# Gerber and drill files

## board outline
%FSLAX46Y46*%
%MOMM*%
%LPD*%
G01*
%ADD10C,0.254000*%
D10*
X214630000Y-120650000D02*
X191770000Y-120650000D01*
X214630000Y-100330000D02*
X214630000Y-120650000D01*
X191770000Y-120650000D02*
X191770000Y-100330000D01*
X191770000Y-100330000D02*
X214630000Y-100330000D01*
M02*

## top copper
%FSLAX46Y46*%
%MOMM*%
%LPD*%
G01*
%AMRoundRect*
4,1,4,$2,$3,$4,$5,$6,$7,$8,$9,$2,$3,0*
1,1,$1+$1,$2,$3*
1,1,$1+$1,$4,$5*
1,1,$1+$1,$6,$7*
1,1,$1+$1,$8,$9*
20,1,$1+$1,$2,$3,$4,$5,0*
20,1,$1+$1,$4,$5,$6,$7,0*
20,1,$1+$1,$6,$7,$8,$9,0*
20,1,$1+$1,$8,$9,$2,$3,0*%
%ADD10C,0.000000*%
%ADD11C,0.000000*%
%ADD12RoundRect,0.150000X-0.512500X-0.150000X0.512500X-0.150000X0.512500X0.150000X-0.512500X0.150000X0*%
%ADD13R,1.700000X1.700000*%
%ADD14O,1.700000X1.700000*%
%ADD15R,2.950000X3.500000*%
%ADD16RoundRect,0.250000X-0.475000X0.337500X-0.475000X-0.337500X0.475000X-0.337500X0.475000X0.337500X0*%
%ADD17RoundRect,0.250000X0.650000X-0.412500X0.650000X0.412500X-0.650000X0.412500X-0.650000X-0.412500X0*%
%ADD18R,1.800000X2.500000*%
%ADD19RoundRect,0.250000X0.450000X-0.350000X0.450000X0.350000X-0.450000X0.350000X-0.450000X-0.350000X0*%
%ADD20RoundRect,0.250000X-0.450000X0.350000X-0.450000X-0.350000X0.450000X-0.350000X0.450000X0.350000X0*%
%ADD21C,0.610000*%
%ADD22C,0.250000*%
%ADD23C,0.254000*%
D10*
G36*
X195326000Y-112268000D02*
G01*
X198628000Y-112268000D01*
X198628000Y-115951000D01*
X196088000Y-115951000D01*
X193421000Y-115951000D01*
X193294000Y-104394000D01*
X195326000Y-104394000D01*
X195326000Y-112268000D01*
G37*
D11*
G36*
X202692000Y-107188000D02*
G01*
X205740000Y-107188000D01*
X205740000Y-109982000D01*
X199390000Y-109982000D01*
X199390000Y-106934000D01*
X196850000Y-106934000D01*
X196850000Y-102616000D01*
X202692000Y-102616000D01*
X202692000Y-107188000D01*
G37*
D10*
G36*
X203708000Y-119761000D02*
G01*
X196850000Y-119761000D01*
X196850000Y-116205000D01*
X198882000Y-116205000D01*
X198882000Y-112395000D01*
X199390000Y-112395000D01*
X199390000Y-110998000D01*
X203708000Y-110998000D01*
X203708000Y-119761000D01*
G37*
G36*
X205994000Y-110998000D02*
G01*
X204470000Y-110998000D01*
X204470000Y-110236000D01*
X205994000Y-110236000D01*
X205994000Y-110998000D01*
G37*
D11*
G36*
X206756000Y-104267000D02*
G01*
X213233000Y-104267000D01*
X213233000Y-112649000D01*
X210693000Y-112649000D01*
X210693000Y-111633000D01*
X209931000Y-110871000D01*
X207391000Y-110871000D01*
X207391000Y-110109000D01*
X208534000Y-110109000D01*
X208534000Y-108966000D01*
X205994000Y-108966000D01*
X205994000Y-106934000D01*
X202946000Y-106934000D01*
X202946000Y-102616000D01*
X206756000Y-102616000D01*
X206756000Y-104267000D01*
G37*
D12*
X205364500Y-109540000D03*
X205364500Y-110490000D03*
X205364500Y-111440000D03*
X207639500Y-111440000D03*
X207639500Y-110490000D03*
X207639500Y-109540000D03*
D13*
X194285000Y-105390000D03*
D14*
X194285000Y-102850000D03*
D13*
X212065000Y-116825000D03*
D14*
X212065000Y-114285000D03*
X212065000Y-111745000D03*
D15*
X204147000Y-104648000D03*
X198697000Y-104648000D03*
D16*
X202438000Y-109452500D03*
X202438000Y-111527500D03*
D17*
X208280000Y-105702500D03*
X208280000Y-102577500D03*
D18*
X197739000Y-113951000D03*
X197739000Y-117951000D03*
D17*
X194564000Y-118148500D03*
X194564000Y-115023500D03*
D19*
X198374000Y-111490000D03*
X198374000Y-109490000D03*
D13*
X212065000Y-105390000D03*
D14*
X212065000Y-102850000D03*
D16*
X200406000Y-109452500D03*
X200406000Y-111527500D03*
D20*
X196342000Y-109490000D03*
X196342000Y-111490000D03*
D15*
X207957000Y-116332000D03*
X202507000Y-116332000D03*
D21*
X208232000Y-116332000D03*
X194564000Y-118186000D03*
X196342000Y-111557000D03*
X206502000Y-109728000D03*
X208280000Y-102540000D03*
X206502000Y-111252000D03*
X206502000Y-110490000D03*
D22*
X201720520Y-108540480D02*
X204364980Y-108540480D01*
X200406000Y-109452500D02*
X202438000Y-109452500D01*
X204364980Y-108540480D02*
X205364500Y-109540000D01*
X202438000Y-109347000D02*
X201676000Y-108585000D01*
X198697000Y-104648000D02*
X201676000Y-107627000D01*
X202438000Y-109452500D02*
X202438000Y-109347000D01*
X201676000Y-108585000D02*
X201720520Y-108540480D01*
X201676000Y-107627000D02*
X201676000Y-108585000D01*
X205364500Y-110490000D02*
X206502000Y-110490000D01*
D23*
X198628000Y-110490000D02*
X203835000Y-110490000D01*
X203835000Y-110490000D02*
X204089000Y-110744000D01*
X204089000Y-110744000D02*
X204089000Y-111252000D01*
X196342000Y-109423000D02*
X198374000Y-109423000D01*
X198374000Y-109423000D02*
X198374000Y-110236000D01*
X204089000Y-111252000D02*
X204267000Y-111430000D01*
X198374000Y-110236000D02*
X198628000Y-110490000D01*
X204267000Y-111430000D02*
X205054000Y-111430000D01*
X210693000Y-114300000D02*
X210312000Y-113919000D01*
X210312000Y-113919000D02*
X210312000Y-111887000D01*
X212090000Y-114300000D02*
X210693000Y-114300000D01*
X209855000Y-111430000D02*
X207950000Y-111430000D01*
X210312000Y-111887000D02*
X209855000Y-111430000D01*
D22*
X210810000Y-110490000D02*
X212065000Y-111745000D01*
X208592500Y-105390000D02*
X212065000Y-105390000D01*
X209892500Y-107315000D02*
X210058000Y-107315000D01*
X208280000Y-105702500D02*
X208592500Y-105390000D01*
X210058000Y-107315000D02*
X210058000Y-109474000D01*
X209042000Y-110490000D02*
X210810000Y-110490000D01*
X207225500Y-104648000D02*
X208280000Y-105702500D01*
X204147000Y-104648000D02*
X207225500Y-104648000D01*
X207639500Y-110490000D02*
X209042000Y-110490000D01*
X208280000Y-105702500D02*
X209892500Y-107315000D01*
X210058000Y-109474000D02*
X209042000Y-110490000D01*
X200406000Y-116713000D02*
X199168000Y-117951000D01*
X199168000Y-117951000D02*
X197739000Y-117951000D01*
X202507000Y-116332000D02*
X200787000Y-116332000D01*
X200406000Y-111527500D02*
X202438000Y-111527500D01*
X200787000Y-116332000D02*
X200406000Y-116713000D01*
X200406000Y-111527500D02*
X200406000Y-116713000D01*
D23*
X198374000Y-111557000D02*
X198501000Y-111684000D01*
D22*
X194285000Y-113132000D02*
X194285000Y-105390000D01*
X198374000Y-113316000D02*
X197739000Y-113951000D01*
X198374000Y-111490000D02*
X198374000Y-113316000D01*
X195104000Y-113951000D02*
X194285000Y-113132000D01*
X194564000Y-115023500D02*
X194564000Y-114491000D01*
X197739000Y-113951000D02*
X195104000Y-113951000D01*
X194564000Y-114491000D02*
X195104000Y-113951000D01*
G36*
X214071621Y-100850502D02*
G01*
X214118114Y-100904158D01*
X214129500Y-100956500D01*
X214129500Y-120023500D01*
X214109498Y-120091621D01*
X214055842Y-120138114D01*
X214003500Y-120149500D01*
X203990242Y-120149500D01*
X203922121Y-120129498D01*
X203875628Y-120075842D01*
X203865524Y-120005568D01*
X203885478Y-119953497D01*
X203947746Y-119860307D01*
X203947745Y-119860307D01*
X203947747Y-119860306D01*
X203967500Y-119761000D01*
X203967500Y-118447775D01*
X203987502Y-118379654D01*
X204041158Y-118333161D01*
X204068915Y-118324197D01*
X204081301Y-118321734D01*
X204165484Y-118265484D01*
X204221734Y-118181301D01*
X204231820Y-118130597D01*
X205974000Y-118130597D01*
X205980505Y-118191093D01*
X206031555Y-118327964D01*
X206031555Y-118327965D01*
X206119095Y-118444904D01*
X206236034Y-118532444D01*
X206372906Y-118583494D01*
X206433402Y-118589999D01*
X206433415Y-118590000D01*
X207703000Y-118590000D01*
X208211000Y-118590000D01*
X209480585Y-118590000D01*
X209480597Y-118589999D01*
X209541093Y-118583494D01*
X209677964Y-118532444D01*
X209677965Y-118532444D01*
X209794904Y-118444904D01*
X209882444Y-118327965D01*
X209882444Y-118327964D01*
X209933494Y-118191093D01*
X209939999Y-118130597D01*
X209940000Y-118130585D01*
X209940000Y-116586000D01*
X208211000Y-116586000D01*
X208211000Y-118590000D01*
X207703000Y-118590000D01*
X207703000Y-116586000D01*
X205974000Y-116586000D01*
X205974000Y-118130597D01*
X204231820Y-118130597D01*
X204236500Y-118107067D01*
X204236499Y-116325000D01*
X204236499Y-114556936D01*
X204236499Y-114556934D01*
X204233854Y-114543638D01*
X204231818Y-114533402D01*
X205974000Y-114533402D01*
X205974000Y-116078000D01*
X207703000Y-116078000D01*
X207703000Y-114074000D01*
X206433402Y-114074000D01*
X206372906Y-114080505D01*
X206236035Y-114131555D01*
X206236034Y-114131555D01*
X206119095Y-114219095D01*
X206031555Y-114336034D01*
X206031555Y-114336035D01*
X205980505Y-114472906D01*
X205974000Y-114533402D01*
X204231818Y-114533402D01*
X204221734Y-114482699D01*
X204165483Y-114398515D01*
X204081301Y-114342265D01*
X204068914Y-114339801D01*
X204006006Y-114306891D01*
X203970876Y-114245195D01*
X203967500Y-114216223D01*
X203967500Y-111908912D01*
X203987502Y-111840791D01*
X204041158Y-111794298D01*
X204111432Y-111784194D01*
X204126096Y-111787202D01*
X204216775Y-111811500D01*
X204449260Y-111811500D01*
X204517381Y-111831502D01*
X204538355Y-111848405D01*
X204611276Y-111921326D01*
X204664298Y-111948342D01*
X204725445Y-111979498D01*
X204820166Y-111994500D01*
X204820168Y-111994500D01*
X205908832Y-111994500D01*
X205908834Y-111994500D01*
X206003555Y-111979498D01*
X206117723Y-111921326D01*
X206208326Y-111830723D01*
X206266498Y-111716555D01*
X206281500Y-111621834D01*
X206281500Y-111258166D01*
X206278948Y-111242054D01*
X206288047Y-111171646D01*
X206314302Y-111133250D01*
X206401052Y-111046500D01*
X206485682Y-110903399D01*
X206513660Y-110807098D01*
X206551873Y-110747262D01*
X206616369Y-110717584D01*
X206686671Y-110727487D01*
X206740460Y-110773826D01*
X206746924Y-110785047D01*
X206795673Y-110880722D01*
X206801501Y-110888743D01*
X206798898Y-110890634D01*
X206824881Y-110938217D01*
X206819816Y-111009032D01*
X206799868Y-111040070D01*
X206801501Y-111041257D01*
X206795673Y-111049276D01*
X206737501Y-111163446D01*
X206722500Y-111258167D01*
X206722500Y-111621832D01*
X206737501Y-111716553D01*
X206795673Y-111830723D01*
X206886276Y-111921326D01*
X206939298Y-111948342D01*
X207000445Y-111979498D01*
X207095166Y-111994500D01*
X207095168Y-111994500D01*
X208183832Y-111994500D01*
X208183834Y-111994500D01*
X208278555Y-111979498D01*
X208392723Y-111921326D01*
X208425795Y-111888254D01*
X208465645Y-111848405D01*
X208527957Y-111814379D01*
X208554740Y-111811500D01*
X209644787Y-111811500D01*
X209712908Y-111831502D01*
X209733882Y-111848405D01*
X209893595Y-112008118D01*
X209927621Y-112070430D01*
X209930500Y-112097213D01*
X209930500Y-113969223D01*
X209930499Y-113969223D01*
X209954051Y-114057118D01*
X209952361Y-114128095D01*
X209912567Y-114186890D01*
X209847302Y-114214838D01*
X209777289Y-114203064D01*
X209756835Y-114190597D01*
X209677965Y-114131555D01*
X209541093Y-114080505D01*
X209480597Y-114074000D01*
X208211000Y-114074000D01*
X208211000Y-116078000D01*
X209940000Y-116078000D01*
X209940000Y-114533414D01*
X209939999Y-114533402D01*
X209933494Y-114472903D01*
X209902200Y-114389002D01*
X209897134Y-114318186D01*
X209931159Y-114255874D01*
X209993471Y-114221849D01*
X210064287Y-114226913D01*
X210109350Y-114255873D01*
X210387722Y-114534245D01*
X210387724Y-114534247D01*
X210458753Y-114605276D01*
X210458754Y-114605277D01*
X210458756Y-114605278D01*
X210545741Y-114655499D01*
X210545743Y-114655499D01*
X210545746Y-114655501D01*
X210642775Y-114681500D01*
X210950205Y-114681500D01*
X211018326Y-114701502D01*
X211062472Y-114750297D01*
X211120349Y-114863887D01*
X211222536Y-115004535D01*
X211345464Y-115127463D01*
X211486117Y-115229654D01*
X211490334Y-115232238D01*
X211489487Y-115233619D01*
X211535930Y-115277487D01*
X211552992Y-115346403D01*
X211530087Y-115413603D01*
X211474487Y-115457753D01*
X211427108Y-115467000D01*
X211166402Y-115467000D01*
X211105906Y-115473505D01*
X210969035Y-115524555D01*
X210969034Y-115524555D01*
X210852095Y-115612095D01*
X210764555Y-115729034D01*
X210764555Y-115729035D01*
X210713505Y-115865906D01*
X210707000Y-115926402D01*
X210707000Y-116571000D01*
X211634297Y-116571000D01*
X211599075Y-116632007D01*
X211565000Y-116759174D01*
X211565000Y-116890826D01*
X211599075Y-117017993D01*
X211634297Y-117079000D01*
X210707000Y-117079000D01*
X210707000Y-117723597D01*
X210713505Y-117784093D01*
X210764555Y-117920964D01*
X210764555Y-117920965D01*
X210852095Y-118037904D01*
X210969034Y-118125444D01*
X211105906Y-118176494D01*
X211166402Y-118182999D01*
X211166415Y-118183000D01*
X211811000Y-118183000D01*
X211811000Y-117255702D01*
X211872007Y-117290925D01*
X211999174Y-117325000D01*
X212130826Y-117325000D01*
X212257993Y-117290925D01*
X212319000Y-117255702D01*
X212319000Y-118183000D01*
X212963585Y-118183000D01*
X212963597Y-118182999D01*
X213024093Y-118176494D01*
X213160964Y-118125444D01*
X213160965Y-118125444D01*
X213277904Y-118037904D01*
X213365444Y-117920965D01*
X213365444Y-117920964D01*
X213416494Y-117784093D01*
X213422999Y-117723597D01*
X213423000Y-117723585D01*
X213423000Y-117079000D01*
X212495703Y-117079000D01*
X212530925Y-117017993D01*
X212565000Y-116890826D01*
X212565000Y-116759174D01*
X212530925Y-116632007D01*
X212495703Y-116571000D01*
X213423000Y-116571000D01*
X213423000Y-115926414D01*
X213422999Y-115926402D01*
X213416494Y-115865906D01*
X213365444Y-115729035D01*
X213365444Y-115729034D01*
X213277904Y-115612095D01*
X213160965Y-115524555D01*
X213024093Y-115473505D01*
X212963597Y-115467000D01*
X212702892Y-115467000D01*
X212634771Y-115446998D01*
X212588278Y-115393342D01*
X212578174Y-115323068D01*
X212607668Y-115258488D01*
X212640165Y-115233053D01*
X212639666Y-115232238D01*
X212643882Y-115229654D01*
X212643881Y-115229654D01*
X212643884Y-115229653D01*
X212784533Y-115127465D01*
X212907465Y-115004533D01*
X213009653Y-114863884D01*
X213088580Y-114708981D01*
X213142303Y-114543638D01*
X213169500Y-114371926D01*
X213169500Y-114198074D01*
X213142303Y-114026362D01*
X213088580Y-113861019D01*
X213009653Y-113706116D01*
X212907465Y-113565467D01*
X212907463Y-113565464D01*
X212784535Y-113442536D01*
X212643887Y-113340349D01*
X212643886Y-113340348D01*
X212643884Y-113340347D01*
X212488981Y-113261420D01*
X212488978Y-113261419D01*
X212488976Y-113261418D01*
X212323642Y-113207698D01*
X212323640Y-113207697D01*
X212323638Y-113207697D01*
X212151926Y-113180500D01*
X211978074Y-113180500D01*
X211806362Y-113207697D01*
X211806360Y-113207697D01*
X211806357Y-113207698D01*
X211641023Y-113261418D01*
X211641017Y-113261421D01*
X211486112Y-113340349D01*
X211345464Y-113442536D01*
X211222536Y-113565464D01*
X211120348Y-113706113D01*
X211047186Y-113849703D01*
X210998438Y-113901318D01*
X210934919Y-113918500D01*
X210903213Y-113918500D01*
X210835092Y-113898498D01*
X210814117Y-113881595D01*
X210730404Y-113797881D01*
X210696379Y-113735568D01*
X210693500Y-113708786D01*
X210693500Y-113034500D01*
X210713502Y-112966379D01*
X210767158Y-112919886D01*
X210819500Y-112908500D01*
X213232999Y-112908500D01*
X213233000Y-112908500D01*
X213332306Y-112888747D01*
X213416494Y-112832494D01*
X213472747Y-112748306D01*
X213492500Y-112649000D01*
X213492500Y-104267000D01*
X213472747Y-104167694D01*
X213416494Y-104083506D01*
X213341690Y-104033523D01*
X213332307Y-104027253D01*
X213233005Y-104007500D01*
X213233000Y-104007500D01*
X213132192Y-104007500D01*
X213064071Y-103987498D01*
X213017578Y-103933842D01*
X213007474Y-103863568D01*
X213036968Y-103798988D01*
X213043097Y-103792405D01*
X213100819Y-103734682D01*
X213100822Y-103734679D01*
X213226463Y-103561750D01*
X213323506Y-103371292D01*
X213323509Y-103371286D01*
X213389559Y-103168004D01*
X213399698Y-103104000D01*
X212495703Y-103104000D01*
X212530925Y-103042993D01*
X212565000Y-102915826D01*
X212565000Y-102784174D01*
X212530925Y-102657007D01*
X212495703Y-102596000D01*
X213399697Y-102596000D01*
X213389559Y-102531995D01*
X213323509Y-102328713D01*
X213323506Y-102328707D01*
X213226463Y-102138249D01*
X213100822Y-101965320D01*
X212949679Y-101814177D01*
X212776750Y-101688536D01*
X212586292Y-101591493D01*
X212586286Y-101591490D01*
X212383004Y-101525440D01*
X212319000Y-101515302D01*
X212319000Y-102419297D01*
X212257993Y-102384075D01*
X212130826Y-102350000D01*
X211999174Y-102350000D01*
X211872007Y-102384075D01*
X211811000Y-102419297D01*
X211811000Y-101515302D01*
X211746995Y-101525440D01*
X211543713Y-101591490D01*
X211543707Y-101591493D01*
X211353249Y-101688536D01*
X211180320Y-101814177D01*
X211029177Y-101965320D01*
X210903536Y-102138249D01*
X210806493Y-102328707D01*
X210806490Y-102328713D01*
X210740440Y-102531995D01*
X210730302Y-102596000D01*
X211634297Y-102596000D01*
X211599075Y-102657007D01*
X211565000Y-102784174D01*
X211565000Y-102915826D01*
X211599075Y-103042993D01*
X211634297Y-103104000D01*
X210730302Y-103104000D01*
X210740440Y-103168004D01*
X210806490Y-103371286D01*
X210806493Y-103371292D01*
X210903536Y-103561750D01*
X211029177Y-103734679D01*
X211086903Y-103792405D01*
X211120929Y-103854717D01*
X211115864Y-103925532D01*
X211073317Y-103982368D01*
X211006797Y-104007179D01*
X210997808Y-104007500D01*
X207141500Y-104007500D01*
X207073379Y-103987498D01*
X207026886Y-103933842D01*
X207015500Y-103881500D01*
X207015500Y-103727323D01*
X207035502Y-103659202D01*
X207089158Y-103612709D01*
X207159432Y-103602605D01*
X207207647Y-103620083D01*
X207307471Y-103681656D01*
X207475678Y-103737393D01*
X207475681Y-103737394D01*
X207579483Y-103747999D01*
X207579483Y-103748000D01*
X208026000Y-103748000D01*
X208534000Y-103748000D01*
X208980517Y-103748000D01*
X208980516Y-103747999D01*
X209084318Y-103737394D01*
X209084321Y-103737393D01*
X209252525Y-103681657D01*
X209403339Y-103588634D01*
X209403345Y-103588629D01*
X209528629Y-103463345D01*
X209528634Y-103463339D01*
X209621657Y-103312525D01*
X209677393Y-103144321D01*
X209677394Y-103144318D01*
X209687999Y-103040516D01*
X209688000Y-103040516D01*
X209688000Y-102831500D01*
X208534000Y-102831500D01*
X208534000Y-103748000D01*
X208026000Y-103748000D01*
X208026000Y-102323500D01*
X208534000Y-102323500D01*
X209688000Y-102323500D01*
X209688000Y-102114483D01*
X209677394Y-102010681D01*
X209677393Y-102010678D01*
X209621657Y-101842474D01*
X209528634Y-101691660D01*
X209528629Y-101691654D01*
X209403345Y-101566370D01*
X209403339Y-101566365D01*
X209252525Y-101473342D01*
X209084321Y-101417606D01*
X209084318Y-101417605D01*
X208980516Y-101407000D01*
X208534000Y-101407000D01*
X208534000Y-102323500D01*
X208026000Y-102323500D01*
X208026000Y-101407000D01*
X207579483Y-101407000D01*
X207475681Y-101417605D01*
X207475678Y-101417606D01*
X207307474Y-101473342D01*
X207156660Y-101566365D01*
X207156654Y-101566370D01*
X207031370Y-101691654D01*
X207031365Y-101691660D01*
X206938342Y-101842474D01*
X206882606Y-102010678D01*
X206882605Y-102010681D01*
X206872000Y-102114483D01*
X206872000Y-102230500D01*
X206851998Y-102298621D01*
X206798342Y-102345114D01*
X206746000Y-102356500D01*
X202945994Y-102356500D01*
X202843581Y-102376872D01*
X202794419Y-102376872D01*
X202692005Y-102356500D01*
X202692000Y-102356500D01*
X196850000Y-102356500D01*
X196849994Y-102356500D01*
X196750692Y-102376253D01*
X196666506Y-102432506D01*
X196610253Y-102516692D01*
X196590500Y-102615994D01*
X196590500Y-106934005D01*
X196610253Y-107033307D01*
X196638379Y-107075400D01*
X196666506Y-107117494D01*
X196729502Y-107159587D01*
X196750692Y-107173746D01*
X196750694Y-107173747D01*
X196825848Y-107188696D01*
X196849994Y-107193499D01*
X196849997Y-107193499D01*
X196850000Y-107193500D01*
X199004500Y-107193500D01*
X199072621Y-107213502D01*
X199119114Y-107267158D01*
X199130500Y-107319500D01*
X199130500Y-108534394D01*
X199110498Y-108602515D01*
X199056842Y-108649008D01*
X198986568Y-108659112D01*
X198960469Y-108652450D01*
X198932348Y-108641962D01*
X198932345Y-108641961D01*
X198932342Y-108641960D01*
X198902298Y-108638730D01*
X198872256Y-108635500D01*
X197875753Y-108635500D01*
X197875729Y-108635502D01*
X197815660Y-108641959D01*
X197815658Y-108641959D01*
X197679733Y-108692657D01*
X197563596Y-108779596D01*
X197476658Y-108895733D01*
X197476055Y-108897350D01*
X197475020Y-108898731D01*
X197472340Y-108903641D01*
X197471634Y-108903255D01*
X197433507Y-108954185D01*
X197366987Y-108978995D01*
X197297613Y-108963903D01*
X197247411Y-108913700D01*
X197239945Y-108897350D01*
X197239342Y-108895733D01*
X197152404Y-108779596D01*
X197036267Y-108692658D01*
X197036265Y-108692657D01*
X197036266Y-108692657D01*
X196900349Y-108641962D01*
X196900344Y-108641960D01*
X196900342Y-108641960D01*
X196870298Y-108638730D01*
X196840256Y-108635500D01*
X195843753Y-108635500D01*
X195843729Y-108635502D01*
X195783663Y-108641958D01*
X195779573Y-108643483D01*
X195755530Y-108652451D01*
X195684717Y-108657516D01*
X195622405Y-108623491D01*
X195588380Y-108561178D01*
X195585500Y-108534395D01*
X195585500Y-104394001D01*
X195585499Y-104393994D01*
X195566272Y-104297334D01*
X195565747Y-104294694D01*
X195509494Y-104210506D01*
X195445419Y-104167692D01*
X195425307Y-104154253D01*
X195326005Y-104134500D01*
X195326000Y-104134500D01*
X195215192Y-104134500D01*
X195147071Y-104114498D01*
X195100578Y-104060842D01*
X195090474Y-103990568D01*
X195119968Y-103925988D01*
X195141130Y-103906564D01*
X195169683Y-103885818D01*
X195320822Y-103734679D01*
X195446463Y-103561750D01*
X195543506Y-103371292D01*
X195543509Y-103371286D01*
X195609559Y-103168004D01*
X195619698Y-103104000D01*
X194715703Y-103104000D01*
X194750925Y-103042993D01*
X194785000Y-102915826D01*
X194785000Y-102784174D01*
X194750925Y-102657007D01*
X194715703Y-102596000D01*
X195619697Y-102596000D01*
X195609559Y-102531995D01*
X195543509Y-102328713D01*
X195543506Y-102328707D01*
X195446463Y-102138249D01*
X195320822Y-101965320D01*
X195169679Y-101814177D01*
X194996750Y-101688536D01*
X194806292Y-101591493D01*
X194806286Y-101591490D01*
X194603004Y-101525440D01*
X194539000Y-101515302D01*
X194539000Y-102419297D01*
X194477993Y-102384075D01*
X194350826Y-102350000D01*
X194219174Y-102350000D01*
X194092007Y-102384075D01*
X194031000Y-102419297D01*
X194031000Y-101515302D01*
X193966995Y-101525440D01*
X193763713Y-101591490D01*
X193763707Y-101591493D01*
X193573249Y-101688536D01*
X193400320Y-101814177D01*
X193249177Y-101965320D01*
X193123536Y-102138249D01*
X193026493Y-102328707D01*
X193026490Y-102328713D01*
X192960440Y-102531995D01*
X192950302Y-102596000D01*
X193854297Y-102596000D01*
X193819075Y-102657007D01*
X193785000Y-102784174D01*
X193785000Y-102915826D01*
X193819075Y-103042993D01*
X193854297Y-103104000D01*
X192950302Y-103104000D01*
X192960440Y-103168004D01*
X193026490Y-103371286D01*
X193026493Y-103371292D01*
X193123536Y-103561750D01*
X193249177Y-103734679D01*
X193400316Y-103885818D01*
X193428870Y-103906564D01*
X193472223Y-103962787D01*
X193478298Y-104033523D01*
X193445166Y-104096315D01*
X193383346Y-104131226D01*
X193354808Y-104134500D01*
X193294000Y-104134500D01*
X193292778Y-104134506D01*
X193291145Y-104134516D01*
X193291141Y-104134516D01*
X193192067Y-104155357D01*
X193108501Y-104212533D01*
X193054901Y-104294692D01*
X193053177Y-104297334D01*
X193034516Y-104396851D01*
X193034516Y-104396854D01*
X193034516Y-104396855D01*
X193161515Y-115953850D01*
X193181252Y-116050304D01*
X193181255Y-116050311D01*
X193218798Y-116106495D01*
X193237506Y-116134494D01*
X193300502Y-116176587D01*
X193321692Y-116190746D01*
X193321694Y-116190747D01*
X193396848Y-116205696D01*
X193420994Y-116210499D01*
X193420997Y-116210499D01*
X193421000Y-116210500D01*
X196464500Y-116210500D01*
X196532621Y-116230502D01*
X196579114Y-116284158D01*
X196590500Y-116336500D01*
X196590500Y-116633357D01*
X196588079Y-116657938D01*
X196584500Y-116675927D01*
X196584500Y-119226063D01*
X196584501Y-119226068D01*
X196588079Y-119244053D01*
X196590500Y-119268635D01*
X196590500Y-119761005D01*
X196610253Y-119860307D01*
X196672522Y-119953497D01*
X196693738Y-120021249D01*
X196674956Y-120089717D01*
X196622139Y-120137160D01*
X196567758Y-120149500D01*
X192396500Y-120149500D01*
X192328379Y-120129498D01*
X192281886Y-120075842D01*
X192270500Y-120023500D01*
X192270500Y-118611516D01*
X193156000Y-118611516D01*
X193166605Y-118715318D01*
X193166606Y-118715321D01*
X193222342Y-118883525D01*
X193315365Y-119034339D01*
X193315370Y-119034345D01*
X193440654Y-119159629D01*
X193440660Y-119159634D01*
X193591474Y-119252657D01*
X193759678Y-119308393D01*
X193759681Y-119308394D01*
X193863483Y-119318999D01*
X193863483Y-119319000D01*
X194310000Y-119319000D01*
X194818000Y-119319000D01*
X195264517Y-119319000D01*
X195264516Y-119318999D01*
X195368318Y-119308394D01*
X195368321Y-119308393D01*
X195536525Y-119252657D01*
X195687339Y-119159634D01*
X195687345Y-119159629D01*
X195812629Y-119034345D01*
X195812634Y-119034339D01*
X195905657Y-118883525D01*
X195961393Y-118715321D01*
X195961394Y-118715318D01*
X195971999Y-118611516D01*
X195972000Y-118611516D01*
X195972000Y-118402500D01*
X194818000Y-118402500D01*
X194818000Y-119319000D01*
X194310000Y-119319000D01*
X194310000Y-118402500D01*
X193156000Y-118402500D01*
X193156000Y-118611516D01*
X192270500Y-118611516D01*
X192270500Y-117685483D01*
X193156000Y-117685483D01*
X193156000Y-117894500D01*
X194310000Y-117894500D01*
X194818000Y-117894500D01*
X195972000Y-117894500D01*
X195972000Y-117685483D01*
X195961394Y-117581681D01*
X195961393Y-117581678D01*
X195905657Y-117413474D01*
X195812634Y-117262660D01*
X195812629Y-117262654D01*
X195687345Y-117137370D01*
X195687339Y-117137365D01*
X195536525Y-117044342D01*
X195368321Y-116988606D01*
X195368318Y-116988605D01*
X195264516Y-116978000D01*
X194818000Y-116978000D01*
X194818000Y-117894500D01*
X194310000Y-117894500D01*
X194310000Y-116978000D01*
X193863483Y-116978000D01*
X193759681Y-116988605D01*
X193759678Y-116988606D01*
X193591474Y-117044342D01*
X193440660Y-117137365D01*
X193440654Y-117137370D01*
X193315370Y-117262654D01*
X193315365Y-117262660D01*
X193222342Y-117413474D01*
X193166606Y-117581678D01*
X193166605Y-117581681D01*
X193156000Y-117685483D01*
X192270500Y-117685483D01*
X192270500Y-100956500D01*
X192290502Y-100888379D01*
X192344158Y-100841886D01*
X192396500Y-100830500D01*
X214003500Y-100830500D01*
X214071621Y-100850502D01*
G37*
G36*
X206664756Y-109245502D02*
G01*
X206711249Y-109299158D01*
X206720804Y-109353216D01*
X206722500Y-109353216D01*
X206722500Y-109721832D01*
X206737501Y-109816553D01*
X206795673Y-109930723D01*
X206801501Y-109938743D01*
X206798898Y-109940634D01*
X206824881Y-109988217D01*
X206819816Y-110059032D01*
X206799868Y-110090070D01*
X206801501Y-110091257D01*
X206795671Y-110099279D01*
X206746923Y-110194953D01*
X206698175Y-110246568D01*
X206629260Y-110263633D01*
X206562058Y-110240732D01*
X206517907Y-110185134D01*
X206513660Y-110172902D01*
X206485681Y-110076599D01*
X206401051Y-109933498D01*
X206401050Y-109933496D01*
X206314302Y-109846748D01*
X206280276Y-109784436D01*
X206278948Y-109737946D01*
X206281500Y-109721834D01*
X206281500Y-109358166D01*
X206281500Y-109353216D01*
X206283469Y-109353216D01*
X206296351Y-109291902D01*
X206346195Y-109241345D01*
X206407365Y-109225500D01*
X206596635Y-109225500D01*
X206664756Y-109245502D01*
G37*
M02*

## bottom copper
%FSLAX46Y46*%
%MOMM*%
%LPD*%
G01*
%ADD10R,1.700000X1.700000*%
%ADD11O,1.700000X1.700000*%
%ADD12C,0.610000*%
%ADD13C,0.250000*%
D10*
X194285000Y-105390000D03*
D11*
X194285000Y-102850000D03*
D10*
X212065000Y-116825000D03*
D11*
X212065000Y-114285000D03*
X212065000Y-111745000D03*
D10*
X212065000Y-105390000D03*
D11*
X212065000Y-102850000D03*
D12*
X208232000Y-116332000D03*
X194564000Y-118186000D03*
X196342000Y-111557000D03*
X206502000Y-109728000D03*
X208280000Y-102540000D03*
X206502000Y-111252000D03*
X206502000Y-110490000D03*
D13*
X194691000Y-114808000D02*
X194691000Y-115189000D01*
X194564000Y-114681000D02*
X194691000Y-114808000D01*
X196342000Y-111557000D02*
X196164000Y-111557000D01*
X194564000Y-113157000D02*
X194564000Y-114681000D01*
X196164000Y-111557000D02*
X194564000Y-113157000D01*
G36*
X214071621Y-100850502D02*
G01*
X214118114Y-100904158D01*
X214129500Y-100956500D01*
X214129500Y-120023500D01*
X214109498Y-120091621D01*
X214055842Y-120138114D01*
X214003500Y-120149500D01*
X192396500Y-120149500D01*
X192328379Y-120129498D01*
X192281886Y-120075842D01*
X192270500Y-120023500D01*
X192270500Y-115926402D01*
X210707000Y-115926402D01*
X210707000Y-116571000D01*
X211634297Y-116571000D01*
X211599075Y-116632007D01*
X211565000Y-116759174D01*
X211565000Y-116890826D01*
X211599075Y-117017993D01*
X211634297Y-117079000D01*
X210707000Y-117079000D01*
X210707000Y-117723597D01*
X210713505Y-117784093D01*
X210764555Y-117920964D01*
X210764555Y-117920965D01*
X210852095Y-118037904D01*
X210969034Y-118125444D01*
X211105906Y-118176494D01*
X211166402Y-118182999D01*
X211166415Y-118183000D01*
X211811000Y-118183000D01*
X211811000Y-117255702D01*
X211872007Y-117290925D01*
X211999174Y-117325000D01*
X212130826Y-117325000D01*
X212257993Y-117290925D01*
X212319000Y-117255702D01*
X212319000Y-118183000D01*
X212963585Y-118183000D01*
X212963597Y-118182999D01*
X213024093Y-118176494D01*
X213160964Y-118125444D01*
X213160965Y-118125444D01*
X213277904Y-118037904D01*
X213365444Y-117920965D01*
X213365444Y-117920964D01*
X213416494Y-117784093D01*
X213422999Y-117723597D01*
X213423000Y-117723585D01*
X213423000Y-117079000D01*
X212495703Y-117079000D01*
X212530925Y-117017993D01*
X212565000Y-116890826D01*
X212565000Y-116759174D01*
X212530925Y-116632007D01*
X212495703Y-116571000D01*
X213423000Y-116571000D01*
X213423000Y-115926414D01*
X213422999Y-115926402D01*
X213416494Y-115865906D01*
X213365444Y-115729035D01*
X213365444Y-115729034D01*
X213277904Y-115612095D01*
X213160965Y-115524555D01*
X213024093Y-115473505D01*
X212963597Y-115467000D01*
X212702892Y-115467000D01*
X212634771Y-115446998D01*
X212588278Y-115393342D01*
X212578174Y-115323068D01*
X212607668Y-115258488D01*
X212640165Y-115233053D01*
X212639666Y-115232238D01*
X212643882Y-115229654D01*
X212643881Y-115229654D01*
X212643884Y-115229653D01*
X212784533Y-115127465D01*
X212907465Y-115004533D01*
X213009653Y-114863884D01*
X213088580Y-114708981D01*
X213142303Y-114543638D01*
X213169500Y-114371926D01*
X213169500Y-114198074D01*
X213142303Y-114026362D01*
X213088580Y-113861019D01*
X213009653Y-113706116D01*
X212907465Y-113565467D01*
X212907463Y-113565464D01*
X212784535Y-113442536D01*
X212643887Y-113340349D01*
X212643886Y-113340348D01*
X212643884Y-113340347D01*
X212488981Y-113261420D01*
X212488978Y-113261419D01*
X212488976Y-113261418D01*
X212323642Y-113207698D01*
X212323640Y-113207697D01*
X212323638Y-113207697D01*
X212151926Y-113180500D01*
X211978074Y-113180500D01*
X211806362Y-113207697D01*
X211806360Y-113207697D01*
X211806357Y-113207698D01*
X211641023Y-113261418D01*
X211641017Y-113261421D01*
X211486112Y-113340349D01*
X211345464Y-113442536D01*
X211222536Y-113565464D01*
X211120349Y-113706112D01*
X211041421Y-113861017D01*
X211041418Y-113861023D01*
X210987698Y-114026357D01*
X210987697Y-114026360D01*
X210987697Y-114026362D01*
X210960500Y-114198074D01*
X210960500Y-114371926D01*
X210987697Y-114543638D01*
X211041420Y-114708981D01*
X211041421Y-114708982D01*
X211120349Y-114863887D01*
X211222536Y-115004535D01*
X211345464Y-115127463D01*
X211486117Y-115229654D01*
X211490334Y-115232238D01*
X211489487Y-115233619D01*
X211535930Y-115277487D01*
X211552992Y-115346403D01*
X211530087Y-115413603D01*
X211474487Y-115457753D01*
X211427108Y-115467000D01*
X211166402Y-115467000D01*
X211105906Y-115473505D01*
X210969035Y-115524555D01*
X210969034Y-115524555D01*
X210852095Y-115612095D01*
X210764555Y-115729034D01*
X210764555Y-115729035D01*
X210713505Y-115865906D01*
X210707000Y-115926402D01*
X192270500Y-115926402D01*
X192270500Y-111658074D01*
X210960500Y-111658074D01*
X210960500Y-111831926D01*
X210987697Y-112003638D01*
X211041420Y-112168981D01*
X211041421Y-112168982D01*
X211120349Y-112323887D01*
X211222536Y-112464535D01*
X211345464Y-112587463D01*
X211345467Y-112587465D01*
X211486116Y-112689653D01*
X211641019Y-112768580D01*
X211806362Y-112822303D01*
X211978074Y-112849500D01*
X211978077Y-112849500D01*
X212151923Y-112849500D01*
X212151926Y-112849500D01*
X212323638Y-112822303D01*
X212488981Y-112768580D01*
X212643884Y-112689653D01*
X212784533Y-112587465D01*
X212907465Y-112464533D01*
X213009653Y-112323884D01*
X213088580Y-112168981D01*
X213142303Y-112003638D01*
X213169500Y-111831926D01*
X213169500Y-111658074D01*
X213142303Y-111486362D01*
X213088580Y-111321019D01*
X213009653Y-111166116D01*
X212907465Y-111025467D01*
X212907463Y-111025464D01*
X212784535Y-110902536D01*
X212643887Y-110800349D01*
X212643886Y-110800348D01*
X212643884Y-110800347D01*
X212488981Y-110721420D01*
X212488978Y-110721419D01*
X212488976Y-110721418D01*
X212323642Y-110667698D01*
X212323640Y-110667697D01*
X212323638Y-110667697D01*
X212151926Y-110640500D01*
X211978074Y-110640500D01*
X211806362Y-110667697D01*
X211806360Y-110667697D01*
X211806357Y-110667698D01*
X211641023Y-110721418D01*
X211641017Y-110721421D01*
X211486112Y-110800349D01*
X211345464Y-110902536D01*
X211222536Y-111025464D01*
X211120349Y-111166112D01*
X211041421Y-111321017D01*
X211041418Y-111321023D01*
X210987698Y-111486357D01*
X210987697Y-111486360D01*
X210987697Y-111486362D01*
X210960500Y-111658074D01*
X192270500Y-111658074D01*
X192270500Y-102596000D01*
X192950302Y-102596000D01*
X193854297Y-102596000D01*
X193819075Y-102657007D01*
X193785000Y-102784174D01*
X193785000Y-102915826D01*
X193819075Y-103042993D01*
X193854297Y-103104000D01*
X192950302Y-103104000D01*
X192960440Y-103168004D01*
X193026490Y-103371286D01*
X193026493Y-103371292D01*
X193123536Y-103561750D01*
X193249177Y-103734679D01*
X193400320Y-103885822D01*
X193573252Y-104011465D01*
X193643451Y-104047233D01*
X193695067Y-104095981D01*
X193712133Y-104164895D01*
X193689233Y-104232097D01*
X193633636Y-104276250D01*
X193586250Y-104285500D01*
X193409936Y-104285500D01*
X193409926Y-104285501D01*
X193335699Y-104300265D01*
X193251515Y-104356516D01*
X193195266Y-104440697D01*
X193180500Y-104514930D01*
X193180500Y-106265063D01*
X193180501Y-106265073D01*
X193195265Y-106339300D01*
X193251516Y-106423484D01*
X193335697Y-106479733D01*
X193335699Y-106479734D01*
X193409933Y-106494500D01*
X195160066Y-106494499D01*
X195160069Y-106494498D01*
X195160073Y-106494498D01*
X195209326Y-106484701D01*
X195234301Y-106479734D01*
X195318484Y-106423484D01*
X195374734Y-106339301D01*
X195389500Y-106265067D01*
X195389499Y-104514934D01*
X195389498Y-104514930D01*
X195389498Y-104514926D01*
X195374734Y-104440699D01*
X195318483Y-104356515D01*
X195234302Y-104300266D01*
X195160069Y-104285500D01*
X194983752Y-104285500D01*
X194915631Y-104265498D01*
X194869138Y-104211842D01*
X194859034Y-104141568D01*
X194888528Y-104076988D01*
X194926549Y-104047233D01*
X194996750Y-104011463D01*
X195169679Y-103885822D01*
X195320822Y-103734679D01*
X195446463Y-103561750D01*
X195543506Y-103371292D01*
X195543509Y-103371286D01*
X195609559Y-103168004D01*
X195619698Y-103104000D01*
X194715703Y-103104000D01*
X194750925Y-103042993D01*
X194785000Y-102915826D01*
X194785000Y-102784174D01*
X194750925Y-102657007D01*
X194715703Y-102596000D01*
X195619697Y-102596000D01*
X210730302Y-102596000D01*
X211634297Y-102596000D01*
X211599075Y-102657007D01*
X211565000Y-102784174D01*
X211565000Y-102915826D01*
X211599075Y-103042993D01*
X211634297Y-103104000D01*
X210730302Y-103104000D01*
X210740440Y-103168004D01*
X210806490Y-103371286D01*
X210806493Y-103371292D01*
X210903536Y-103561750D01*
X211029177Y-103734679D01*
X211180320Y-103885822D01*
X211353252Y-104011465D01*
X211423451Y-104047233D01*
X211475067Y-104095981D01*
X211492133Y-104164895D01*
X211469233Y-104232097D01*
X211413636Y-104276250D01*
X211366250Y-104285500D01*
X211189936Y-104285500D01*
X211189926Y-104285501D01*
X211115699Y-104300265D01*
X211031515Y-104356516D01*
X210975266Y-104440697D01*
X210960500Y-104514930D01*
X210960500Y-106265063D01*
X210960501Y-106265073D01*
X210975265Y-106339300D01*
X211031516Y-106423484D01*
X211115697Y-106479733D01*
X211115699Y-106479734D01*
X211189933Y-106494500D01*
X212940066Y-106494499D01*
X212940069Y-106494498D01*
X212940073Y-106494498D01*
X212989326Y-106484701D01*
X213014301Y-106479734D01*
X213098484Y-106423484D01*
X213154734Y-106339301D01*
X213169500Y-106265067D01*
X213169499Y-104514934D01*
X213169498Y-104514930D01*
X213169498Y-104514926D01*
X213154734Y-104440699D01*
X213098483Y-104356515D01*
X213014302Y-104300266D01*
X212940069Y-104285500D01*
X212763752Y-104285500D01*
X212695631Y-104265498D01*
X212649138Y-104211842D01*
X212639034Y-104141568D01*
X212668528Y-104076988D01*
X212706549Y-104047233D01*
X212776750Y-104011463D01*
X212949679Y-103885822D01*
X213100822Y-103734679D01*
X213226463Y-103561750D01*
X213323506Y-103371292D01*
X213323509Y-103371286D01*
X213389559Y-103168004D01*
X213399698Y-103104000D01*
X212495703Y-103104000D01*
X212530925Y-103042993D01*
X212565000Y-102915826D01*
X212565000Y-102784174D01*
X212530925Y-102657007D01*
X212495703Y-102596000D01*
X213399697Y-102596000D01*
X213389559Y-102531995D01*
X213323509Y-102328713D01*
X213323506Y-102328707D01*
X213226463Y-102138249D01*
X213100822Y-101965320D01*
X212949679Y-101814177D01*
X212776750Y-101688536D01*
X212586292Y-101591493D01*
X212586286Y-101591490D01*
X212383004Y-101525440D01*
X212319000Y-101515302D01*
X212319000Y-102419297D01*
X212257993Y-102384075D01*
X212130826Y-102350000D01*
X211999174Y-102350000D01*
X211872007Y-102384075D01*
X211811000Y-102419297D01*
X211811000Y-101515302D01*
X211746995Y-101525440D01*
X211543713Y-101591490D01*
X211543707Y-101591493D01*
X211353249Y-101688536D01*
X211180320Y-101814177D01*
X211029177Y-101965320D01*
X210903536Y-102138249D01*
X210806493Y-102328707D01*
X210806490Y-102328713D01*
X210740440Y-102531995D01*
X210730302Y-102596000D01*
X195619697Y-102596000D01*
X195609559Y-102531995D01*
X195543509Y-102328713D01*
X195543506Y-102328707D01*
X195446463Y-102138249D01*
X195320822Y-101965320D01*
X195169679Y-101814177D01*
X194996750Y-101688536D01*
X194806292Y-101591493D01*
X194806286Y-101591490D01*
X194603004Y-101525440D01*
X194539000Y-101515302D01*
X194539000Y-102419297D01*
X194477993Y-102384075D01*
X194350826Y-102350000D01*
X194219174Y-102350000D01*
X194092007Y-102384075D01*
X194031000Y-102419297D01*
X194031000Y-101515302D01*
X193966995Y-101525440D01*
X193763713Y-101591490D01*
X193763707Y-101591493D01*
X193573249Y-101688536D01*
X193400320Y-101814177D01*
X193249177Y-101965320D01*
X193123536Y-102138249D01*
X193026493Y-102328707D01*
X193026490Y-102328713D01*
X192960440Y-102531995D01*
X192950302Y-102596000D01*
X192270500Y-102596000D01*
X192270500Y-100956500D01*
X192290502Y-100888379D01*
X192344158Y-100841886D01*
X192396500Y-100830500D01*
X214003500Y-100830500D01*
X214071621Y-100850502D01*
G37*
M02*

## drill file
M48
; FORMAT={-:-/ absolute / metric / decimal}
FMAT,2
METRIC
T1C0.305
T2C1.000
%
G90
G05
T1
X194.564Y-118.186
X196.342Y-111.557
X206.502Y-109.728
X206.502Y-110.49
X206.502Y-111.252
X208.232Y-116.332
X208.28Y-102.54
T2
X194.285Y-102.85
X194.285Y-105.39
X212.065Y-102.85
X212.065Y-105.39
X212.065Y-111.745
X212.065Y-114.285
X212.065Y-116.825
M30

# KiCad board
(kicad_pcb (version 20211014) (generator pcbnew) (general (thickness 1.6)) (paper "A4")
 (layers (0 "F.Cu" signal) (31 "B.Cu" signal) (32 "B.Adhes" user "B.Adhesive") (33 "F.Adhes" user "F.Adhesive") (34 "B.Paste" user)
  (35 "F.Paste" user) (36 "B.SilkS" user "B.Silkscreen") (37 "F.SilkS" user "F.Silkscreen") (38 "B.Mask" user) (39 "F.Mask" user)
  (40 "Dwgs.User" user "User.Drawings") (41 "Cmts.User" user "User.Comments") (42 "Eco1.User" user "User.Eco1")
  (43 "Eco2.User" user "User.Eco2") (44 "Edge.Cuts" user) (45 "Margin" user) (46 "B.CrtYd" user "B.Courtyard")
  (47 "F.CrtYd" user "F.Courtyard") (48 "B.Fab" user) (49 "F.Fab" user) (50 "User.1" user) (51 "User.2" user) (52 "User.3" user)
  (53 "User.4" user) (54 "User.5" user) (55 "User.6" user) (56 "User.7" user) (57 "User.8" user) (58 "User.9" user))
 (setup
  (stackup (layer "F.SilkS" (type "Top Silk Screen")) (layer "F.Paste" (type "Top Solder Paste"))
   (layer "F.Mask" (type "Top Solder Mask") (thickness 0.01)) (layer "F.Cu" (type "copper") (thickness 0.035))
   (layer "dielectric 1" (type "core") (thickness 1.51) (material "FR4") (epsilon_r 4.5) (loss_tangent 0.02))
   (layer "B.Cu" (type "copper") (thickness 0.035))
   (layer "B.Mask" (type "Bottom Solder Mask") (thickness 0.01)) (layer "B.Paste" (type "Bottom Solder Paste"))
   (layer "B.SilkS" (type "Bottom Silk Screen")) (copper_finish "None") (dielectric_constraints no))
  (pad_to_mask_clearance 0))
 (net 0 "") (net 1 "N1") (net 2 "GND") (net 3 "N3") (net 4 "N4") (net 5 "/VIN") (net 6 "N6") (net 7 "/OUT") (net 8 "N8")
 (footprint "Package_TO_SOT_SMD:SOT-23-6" (layer "F.Cu") (at 206.502 110.49)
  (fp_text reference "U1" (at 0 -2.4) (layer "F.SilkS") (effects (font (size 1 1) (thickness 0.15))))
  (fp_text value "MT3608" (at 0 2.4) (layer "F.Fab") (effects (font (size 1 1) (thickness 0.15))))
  (pad "1" smd roundrect locked (at -1.1375 -0.95) (size 1.325 0.6) (layers "F.Cu" "F.Paste" "F.Mask") (roundrect_rratio 0.25) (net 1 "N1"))
  (pad "2" smd roundrect locked (at -1.1375 0) (size 1.325 0.6) (layers "F.Cu" "F.Paste" "F.Mask") (roundrect_rratio 0.25) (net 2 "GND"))
  (pad "3" smd roundrect locked (at -1.1375 0.95) (size 1.325 0.6) (layers "F.Cu" "F.Paste" "F.Mask") (roundrect_rratio 0.25) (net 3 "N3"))
  (pad "4" smd roundrect locked (at 1.1375 0.95) (size 1.325 0.6) (layers "F.Cu" "F.Paste" "F.Mask") (roundrect_rratio 0.25) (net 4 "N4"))
  (pad "5" smd roundrect locked (at 1.1375 0) (size 1.325 0.6) (layers "F.Cu" "F.Paste" "F.Mask") (roundrect_rratio 0.25) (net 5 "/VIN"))
  (pad "6" smd roundrect locked (at 1.1375 -0.95) (size 1.325 0.6) (layers "F.Cu" "F.Paste" "F.Mask") (roundrect_rratio 0.25) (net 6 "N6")))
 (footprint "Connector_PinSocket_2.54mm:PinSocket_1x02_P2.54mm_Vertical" (layer "F.Cu") (at 194.285 105.39 180)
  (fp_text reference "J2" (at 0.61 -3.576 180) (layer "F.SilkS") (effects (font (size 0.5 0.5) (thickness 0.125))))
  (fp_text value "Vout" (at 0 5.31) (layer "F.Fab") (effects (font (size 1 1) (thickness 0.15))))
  (pad "1" thru_hole rect locked (at 0 0 180) (size 1.7 1.7) (drill 1) (layers *.Cu *.Mask) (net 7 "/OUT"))
  (pad "2" thru_hole oval locked (at 0 2.54 180) (size 1.7 1.7) (drill 1) (layers *.Cu *.Mask) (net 2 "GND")))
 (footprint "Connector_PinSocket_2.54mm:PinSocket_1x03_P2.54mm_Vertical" (layer "F.Cu") (at 212.065 116.825 180)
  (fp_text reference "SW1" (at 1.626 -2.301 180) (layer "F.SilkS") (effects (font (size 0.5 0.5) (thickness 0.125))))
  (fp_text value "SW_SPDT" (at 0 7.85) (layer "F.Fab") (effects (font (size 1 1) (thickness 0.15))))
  (pad "1" thru_hole rect locked (at 0 0 180) (size 1.7 1.7) (drill 1) (layers *.Cu *.Mask) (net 2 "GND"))
  (pad "2" thru_hole oval locked (at 0 2.54 180) (size 1.7 1.7) (drill 1) (layers *.Cu *.Mask) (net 4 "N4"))
  (pad "3" thru_hole oval locked (at 0 5.08 180) (size 1.7 1.7) (drill 1) (layers *.Cu *.Mask) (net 5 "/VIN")))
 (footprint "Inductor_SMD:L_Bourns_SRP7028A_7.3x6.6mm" (layer "F.Cu") (at 201.422 104.648 180)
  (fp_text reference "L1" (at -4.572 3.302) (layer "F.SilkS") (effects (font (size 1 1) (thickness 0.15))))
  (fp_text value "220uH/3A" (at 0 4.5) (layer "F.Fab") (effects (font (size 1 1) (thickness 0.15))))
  (pad "1" smd rect locked (at -2.725 0 180) (size 2.95 3.5) (layers "F.Cu" "F.Paste" "F.Mask") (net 5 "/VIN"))
  (pad "2" smd rect locked (at 2.725 0 180) (size 2.95 3.5) (layers "F.Cu" "F.Paste" "F.Mask") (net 1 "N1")))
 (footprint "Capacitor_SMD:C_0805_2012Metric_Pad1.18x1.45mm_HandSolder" (layer "F.Cu") (at 202.438 110.49 -90)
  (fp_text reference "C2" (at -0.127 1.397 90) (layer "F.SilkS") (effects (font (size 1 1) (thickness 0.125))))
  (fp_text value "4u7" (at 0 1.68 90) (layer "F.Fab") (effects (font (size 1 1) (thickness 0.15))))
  (pad "1" smd roundrect locked (at -1.0375 0 270) (size 1.175 1.45) (layers "F.Cu" "F.Paste" "F.Mask") (roundrect_rratio 0.212766)
   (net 1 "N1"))
  (pad "2" smd roundrect locked (at 1.0375 0 270) (size 1.175 1.45) (layers "F.Cu" "F.Paste" "F.Mask") (roundrect_rratio 0.212766)
   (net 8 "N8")))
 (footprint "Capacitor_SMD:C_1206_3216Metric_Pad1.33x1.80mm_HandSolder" (layer "F.Cu") (at 208.28 104.14 90)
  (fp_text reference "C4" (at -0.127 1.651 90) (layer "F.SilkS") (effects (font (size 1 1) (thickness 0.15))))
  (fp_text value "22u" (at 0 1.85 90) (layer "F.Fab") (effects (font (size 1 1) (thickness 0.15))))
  (pad "1" smd roundrect locked (at -1.5625 0 90) (size 1.325 1.8) (layers "F.Cu" "F.Paste" "F.Mask") (roundrect_rratio 0.188679)
   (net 5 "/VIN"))
  (pad "2" smd roundrect locked (at 1.5625 0 90) (size 1.325 1.8) (layers "F.Cu" "F.Paste" "F.Mask") (roundrect_rratio 0.188679)
   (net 2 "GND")))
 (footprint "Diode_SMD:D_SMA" (layer "F.Cu") (at 197.739 115.951 -90)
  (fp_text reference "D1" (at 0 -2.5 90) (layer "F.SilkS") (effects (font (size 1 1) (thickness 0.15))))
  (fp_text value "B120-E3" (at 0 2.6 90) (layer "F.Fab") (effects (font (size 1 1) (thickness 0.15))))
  (pad "1" smd rect locked (at -2 0 270) (size 2.5 1.8) (layers "F.Cu" "F.Paste" "F.Mask") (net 7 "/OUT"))
  (pad "2" smd rect locked (at 2 0 270) (size 2.5 1.8) (layers "F.Cu" "F.Paste" "F.Mask") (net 8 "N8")))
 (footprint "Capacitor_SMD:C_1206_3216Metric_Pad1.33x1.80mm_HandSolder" (layer "F.Cu") (at 194.564 116.586 90)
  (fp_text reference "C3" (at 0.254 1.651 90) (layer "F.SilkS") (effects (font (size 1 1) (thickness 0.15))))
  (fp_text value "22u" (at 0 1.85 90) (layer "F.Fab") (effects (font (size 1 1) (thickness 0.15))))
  (pad "1" smd roundrect locked (at -1.5625 0 90) (size 1.325 1.8) (layers "F.Cu" "F.Paste" "F.Mask") (roundrect_rratio 0.188679)
   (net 2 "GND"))
  (pad "2" smd roundrect locked (at 1.5625 0 90) (size 1.325 1.8) (layers "F.Cu" "F.Paste" "F.Mask") (roundrect_rratio 0.188679)
   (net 7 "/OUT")))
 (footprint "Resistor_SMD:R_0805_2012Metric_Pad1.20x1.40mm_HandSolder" (layer "F.Cu") (at 198.374 110.49 90)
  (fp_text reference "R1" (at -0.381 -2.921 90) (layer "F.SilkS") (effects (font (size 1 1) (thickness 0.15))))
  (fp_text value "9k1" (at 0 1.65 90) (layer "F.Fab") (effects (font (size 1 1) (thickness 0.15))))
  (pad "1" smd roundrect locked (at -1 0 90) (size 1.2 1.4) (layers "F.Cu" "F.Paste" "F.Mask") (roundrect_rratio 0.208333) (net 7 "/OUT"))
  (pad "2" smd roundrect locked (at 1 0 90) (size 1.2 1.4) (layers "F.Cu" "F.Paste" "F.Mask") (roundrect_rratio 0.208333) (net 3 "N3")))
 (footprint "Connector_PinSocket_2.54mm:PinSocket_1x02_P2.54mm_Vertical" (layer "F.Cu") (at 212.065 105.39 180)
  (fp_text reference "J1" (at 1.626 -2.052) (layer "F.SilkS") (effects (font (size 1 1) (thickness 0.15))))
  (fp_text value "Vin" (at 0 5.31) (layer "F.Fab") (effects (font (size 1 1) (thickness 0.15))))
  (pad "1" thru_hole rect locked (at 0 0 180) (size 1.7 1.7) (drill 1) (layers *.Cu *.Mask) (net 5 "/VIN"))
  (pad "2" thru_hole oval locked (at 0 2.54 180) (size 1.7 1.7) (drill 1) (layers *.Cu *.Mask) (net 2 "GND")))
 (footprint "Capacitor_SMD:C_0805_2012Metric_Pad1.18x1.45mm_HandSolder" (layer "F.Cu") (at 200.406 110.49 -90)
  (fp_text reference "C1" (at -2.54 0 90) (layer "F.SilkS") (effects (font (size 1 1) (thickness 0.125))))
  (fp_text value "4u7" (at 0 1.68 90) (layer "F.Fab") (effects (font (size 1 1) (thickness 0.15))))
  (pad "1" smd roundrect locked (at -1.0375 0 270) (size 1.175 1.45) (layers "F.Cu" "F.Paste" "F.Mask") (roundrect_rratio 0.212766)
   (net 1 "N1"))
  (pad "2" smd roundrect locked (at 1.0375 0 270) (size 1.175 1.45) (layers "F.Cu" "F.Paste" "F.Mask") (roundrect_rratio 0.212766)
   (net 8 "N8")))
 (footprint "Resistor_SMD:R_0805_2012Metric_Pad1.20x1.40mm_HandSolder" (layer "F.Cu") (at 196.342 110.49 -90)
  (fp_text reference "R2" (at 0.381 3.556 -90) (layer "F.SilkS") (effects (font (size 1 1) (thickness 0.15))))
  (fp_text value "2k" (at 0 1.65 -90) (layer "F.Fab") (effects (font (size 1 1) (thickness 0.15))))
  (pad "1" smd roundrect locked (at -1 0 270) (size 1.2 1.4) (layers "F.Cu" "F.Paste" "F.Mask") (roundrect_rratio 0.208333) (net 3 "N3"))
  (pad "2" smd roundrect locked (at 1 0 270) (size 1.2 1.4) (layers "F.Cu" "F.Paste" "F.Mask") (roundrect_rratio 0.208333) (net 2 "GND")))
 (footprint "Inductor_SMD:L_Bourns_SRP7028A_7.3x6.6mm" (layer "F.Cu") (at 205.232 116.332 180)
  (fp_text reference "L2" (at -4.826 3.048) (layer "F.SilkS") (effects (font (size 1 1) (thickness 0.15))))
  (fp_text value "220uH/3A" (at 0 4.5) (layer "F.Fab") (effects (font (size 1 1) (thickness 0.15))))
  (pad "1" smd rect locked (at -2.725 0 180) (size 2.95 3.5) (layers "F.Cu" "F.Paste" "F.Mask") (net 2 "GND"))
  (pad "2" smd rect locked (at 2.725 0 180) (size 2.95 3.5) (layers "F.Cu" "F.Paste" "F.Mask") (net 8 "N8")))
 (gr_poly
  (pts (xy 198.628 115.951) (xy 198.628 112.268) (xy 195.326 112.268) (xy 195.326 104.394) (xy 193.294 104.394) (xy 193.421 115.951)
   (xy 196.088 115.951))
  (layer "F.Cu") (width 0) (fill solid))
 (gr_poly
  (pts (xy 196.85 102.616) (xy 196.85 106.934) (xy 199.39 106.934) (xy 199.39 109.982) (xy 205.74 109.982) (xy 205.74 107.188)
   (xy 202.692 107.188) (xy 202.692 102.616))
  (layer "F.Cu") (width 0) (fill solid))
 (gr_poly
  (pts (xy 199.39 110.998) (xy 199.39 112.395) (xy 198.882 112.395) (xy 198.882 116.205) (xy 196.85 116.205) (xy 196.85 119.761)
   (xy 203.708 119.761) (xy 203.708 110.998))
  (layer "F.Cu") (width 0) (fill solid))
 (gr_poly (pts (xy 204.47 110.236) (xy 205.994 110.236) (xy 205.994 110.998) (xy 204.47 110.998)) (layer "F.Cu") (width 0) (fill solid))
 (gr_poly
  (pts (xy 213.233 104.267) (xy 206.756 104.267) (xy 206.756 102.616) (xy 202.946 102.616) (xy 202.946 106.934) (xy 205.994 106.934)
   (xy 205.994 108.966) (xy 208.534 108.966) (xy 208.534 110.109) (xy 207.391 110.109) (xy 207.391 110.871) (xy 209.931 110.871)
   (xy 210.693 111.633) (xy 210.693 112.649) (xy 213.233 112.649))
  (layer "F.Cu") (width 0) (fill solid))
 (gr_line (start 214.63 120.65) (end 191.77 120.65) (layer "Edge.Cuts") (width 0.254))
 (gr_line (start 214.63 100.33) (end 214.63 120.65) (layer "Edge.Cuts") (width 0.254))
 (gr_line (start 191.77 120.65) (end 191.77 100.33) (layer "Edge.Cuts") (width 0.254))
 (gr_line (start 191.77 100.33) (end 214.63 100.33) (layer "Edge.Cuts") (width 0.254))
 (segment (start 201.72052 108.54048) (end 204.36498 108.54048) (width 0.25) (layer "F.Cu") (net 1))
 (segment (start 200.406 109.4525) (end 202.438 109.4525) (width 0.25) (layer "F.Cu") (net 1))
 (segment (start 204.36498 108.54048) (end 205.3645 109.54) (width 0.25) (layer "F.Cu") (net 1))
 (segment (start 202.438 109.347) (end 201.676 108.585) (width 0.25) (layer "F.Cu") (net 1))
 (segment (start 198.697 104.648) (end 201.676 107.627) (width 0.25) (layer "F.Cu") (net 1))
 (segment (start 202.438 109.4525) (end 202.438 109.347) (width 0.25) (layer "F.Cu") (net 1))
 (segment (start 201.676 108.585) (end 201.72052 108.54048) (width 0.25) (layer "F.Cu") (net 1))
 (segment (start 201.676 107.627) (end 201.676 108.585) (width 0.25) (layer "F.Cu") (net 1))
 (segment (start 205.3645 110.49) (end 206.502 110.49) (width 0.25) (layer "F.Cu") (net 2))
 (via (at 208.232 116.332) (size 0.61) (drill 0.305) (layers "F.Cu" "B.Cu") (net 2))
 (via (at 194.564 118.186) (size 0.61) (drill 0.305) (layers "F.Cu" "B.Cu") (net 2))
 (via (at 196.342 111.557) (size 0.61) (drill 0.305) (layers "F.Cu" "B.Cu") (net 2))
 (via (at 206.502 109.728) (size 0.61) (drill 0.305) (layers "F.Cu" "B.Cu") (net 2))
 (via (at 208.28 102.54) (size 0.61) (drill 0.305) (layers "F.Cu" "B.Cu") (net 2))
 (via (at 206.502 111.252) (size 0.61) (drill 0.305) (layers "F.Cu" "B.Cu") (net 2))
 (via (at 206.502 110.49) (size 0.61) (drill 0.305) (layers "F.Cu" "B.Cu") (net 2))
 (segment (start 194.691 114.808) (end 194.691 115.189) (width 0.25) (layer "B.Cu") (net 2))
 (segment (start 194.564 114.681) (end 194.691 114.808) (width 0.25) (layer "B.Cu") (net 2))
 (segment (start 196.342 111.557) (end 196.164 111.557) (width 0.25) (layer "B.Cu") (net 2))
 (segment (start 194.564 113.157) (end 194.564 114.681) (width 0.25) (layer "B.Cu") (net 2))
 (segment (start 196.164 111.557) (end 194.564 113.157) (width 0.25) (layer "B.Cu") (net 2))
 (segment (start 198.628 110.49) (end 203.835 110.49) (width 0.254) (layer "F.Cu") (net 3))
 (segment (start 203.835 110.49) (end 204.089 110.744) (width 0.254) (layer "F.Cu") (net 3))
 (segment (start 204.089 110.744) (end 204.089 111.252) (width 0.254) (layer "F.Cu") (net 3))
 (segment (start 196.342 109.423) (end 198.374 109.423) (width 0.254) (layer "F.Cu") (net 3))
 (segment (start 198.374 109.423) (end 198.374 110.236) (width 0.254) (layer "F.Cu") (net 3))
 (segment (start 204.089 111.252) (end 204.267 111.43) (width 0.254) (layer "F.Cu") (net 3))
 (segment (start 198.374 110.236) (end 198.628 110.49) (width 0.254) (layer "F.Cu") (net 3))
 (segment (start 204.267 111.43) (end 205.054 111.43) (width 0.254) (layer "F.Cu") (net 3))
 (segment (start 210.693 114.3) (end 210.312 113.919) (width 0.254) (layer "F.Cu") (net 4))
 (segment (start 210.312 113.919) (end 210.312 111.887) (width 0.254) (layer "F.Cu") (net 4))
 (segment (start 212.09 114.3) (end 210.693 114.3) (width 0.254) (layer "F.Cu") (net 4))
 (segment (start 209.855 111.43) (end 207.95 111.43) (width 0.254) (layer "F.Cu") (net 4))
 (segment (start 210.312 111.887) (end 209.855 111.43) (width 0.254) (layer "F.Cu") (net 4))
 (segment (start 210.81 110.49) (end 212.065 111.745) (width 0.25) (layer "F.Cu") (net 5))
 (segment (start 208.5925 105.39) (end 212.065 105.39) (width 0.25) (layer "F.Cu") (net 5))
 (segment (start 209.8925 107.315) (end 210.058 107.315) (width 0.25) (layer "F.Cu") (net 5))
 (segment (start 208.28 105.7025) (end 208.5925 105.39) (width 0.25) (layer "F.Cu") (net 5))
 (segment (start 210.058 107.315) (end 210.058 109.474) (width 0.25) (layer "F.Cu") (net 5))
 (segment (start 209.042 110.49) (end 210.81 110.49) (width 0.25) (layer "F.Cu") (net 5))
 (segment (start 207.2255 104.648) (end 208.28 105.7025) (width 0.25) (layer "F.Cu") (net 5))
 (segment (start 204.147 104.648) (end 207.2255 104.648) (width 0.25) (layer "F.Cu") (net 5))
 (segment (start 207.6395 110.49) (end 209.042 110.49) (width 0.25) (layer "F.Cu") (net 5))
 (segment (start 208.28 105.7025) (end 209.8925 107.315) (width 0.25) (layer "F.Cu") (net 5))
 (segment (start 210.058 109.474) (end 209.042 110.49) (width 0.25) (layer "F.Cu") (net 5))
 (segment (start 200.406 116.713) (end 199.168 117.951) (width 0.25) (layer "F.Cu") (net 8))
 (segment (start 199.168 117.951) (end 197.739 117.951) (width 0.25) (layer "F.Cu") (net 8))
 (segment (start 202.507 116.332) (end 200.787 116.332) (width 0.25) (layer "F.Cu") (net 8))
 (segment (start 200.406 111.5275) (end 202.438 111.5275) (width 0.25) (layer "F.Cu") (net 8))
 (segment (start 200.787 116.332) (end 200.406 116.713) (width 0.25) (layer "F.Cu") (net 8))
 (segment (start 200.406 111.5275) (end 200.406 116.713) (width 0.25) (layer "F.Cu") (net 8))
 (segment (start 198.374 111.557) (end 198.501 111.684) (width 0.254) (layer "F.Cu") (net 7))
 (segment (start 194.285 113.132) (end 194.285 105.39) (width 0.25) (layer "F.Cu") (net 7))
 (segment (start 198.374 113.316) (end 197.739 113.951) (width 0.25) (layer "F.Cu") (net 7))
 (segment (start 198.374 111.49) (end 198.374 113.316) (width 0.25) (layer "F.Cu") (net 7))
 (segment (start 195.104 113.951) (end 194.285 113.132) (width 0.25) (layer "F.Cu") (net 7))
 (segment (start 194.564 115.0235) (end 194.564 114.491) (width 0.25) (layer "F.Cu") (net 7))
 (segment (start 197.739 113.951) (end 195.104 113.951) (width 0.25) (layer "F.Cu") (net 7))
 (segment (start 194.564 114.491) (end 195.104 113.951) (width 0.25) (layer "F.Cu") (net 7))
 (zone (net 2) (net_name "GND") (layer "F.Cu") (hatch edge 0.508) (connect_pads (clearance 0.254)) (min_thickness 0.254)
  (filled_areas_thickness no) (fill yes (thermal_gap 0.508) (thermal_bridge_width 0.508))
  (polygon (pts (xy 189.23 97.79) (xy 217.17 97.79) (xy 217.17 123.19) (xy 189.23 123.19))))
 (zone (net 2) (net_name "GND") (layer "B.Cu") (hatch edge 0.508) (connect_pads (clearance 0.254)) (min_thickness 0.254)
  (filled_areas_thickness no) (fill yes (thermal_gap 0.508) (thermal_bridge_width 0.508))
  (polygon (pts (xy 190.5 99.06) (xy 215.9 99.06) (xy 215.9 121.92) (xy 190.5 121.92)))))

